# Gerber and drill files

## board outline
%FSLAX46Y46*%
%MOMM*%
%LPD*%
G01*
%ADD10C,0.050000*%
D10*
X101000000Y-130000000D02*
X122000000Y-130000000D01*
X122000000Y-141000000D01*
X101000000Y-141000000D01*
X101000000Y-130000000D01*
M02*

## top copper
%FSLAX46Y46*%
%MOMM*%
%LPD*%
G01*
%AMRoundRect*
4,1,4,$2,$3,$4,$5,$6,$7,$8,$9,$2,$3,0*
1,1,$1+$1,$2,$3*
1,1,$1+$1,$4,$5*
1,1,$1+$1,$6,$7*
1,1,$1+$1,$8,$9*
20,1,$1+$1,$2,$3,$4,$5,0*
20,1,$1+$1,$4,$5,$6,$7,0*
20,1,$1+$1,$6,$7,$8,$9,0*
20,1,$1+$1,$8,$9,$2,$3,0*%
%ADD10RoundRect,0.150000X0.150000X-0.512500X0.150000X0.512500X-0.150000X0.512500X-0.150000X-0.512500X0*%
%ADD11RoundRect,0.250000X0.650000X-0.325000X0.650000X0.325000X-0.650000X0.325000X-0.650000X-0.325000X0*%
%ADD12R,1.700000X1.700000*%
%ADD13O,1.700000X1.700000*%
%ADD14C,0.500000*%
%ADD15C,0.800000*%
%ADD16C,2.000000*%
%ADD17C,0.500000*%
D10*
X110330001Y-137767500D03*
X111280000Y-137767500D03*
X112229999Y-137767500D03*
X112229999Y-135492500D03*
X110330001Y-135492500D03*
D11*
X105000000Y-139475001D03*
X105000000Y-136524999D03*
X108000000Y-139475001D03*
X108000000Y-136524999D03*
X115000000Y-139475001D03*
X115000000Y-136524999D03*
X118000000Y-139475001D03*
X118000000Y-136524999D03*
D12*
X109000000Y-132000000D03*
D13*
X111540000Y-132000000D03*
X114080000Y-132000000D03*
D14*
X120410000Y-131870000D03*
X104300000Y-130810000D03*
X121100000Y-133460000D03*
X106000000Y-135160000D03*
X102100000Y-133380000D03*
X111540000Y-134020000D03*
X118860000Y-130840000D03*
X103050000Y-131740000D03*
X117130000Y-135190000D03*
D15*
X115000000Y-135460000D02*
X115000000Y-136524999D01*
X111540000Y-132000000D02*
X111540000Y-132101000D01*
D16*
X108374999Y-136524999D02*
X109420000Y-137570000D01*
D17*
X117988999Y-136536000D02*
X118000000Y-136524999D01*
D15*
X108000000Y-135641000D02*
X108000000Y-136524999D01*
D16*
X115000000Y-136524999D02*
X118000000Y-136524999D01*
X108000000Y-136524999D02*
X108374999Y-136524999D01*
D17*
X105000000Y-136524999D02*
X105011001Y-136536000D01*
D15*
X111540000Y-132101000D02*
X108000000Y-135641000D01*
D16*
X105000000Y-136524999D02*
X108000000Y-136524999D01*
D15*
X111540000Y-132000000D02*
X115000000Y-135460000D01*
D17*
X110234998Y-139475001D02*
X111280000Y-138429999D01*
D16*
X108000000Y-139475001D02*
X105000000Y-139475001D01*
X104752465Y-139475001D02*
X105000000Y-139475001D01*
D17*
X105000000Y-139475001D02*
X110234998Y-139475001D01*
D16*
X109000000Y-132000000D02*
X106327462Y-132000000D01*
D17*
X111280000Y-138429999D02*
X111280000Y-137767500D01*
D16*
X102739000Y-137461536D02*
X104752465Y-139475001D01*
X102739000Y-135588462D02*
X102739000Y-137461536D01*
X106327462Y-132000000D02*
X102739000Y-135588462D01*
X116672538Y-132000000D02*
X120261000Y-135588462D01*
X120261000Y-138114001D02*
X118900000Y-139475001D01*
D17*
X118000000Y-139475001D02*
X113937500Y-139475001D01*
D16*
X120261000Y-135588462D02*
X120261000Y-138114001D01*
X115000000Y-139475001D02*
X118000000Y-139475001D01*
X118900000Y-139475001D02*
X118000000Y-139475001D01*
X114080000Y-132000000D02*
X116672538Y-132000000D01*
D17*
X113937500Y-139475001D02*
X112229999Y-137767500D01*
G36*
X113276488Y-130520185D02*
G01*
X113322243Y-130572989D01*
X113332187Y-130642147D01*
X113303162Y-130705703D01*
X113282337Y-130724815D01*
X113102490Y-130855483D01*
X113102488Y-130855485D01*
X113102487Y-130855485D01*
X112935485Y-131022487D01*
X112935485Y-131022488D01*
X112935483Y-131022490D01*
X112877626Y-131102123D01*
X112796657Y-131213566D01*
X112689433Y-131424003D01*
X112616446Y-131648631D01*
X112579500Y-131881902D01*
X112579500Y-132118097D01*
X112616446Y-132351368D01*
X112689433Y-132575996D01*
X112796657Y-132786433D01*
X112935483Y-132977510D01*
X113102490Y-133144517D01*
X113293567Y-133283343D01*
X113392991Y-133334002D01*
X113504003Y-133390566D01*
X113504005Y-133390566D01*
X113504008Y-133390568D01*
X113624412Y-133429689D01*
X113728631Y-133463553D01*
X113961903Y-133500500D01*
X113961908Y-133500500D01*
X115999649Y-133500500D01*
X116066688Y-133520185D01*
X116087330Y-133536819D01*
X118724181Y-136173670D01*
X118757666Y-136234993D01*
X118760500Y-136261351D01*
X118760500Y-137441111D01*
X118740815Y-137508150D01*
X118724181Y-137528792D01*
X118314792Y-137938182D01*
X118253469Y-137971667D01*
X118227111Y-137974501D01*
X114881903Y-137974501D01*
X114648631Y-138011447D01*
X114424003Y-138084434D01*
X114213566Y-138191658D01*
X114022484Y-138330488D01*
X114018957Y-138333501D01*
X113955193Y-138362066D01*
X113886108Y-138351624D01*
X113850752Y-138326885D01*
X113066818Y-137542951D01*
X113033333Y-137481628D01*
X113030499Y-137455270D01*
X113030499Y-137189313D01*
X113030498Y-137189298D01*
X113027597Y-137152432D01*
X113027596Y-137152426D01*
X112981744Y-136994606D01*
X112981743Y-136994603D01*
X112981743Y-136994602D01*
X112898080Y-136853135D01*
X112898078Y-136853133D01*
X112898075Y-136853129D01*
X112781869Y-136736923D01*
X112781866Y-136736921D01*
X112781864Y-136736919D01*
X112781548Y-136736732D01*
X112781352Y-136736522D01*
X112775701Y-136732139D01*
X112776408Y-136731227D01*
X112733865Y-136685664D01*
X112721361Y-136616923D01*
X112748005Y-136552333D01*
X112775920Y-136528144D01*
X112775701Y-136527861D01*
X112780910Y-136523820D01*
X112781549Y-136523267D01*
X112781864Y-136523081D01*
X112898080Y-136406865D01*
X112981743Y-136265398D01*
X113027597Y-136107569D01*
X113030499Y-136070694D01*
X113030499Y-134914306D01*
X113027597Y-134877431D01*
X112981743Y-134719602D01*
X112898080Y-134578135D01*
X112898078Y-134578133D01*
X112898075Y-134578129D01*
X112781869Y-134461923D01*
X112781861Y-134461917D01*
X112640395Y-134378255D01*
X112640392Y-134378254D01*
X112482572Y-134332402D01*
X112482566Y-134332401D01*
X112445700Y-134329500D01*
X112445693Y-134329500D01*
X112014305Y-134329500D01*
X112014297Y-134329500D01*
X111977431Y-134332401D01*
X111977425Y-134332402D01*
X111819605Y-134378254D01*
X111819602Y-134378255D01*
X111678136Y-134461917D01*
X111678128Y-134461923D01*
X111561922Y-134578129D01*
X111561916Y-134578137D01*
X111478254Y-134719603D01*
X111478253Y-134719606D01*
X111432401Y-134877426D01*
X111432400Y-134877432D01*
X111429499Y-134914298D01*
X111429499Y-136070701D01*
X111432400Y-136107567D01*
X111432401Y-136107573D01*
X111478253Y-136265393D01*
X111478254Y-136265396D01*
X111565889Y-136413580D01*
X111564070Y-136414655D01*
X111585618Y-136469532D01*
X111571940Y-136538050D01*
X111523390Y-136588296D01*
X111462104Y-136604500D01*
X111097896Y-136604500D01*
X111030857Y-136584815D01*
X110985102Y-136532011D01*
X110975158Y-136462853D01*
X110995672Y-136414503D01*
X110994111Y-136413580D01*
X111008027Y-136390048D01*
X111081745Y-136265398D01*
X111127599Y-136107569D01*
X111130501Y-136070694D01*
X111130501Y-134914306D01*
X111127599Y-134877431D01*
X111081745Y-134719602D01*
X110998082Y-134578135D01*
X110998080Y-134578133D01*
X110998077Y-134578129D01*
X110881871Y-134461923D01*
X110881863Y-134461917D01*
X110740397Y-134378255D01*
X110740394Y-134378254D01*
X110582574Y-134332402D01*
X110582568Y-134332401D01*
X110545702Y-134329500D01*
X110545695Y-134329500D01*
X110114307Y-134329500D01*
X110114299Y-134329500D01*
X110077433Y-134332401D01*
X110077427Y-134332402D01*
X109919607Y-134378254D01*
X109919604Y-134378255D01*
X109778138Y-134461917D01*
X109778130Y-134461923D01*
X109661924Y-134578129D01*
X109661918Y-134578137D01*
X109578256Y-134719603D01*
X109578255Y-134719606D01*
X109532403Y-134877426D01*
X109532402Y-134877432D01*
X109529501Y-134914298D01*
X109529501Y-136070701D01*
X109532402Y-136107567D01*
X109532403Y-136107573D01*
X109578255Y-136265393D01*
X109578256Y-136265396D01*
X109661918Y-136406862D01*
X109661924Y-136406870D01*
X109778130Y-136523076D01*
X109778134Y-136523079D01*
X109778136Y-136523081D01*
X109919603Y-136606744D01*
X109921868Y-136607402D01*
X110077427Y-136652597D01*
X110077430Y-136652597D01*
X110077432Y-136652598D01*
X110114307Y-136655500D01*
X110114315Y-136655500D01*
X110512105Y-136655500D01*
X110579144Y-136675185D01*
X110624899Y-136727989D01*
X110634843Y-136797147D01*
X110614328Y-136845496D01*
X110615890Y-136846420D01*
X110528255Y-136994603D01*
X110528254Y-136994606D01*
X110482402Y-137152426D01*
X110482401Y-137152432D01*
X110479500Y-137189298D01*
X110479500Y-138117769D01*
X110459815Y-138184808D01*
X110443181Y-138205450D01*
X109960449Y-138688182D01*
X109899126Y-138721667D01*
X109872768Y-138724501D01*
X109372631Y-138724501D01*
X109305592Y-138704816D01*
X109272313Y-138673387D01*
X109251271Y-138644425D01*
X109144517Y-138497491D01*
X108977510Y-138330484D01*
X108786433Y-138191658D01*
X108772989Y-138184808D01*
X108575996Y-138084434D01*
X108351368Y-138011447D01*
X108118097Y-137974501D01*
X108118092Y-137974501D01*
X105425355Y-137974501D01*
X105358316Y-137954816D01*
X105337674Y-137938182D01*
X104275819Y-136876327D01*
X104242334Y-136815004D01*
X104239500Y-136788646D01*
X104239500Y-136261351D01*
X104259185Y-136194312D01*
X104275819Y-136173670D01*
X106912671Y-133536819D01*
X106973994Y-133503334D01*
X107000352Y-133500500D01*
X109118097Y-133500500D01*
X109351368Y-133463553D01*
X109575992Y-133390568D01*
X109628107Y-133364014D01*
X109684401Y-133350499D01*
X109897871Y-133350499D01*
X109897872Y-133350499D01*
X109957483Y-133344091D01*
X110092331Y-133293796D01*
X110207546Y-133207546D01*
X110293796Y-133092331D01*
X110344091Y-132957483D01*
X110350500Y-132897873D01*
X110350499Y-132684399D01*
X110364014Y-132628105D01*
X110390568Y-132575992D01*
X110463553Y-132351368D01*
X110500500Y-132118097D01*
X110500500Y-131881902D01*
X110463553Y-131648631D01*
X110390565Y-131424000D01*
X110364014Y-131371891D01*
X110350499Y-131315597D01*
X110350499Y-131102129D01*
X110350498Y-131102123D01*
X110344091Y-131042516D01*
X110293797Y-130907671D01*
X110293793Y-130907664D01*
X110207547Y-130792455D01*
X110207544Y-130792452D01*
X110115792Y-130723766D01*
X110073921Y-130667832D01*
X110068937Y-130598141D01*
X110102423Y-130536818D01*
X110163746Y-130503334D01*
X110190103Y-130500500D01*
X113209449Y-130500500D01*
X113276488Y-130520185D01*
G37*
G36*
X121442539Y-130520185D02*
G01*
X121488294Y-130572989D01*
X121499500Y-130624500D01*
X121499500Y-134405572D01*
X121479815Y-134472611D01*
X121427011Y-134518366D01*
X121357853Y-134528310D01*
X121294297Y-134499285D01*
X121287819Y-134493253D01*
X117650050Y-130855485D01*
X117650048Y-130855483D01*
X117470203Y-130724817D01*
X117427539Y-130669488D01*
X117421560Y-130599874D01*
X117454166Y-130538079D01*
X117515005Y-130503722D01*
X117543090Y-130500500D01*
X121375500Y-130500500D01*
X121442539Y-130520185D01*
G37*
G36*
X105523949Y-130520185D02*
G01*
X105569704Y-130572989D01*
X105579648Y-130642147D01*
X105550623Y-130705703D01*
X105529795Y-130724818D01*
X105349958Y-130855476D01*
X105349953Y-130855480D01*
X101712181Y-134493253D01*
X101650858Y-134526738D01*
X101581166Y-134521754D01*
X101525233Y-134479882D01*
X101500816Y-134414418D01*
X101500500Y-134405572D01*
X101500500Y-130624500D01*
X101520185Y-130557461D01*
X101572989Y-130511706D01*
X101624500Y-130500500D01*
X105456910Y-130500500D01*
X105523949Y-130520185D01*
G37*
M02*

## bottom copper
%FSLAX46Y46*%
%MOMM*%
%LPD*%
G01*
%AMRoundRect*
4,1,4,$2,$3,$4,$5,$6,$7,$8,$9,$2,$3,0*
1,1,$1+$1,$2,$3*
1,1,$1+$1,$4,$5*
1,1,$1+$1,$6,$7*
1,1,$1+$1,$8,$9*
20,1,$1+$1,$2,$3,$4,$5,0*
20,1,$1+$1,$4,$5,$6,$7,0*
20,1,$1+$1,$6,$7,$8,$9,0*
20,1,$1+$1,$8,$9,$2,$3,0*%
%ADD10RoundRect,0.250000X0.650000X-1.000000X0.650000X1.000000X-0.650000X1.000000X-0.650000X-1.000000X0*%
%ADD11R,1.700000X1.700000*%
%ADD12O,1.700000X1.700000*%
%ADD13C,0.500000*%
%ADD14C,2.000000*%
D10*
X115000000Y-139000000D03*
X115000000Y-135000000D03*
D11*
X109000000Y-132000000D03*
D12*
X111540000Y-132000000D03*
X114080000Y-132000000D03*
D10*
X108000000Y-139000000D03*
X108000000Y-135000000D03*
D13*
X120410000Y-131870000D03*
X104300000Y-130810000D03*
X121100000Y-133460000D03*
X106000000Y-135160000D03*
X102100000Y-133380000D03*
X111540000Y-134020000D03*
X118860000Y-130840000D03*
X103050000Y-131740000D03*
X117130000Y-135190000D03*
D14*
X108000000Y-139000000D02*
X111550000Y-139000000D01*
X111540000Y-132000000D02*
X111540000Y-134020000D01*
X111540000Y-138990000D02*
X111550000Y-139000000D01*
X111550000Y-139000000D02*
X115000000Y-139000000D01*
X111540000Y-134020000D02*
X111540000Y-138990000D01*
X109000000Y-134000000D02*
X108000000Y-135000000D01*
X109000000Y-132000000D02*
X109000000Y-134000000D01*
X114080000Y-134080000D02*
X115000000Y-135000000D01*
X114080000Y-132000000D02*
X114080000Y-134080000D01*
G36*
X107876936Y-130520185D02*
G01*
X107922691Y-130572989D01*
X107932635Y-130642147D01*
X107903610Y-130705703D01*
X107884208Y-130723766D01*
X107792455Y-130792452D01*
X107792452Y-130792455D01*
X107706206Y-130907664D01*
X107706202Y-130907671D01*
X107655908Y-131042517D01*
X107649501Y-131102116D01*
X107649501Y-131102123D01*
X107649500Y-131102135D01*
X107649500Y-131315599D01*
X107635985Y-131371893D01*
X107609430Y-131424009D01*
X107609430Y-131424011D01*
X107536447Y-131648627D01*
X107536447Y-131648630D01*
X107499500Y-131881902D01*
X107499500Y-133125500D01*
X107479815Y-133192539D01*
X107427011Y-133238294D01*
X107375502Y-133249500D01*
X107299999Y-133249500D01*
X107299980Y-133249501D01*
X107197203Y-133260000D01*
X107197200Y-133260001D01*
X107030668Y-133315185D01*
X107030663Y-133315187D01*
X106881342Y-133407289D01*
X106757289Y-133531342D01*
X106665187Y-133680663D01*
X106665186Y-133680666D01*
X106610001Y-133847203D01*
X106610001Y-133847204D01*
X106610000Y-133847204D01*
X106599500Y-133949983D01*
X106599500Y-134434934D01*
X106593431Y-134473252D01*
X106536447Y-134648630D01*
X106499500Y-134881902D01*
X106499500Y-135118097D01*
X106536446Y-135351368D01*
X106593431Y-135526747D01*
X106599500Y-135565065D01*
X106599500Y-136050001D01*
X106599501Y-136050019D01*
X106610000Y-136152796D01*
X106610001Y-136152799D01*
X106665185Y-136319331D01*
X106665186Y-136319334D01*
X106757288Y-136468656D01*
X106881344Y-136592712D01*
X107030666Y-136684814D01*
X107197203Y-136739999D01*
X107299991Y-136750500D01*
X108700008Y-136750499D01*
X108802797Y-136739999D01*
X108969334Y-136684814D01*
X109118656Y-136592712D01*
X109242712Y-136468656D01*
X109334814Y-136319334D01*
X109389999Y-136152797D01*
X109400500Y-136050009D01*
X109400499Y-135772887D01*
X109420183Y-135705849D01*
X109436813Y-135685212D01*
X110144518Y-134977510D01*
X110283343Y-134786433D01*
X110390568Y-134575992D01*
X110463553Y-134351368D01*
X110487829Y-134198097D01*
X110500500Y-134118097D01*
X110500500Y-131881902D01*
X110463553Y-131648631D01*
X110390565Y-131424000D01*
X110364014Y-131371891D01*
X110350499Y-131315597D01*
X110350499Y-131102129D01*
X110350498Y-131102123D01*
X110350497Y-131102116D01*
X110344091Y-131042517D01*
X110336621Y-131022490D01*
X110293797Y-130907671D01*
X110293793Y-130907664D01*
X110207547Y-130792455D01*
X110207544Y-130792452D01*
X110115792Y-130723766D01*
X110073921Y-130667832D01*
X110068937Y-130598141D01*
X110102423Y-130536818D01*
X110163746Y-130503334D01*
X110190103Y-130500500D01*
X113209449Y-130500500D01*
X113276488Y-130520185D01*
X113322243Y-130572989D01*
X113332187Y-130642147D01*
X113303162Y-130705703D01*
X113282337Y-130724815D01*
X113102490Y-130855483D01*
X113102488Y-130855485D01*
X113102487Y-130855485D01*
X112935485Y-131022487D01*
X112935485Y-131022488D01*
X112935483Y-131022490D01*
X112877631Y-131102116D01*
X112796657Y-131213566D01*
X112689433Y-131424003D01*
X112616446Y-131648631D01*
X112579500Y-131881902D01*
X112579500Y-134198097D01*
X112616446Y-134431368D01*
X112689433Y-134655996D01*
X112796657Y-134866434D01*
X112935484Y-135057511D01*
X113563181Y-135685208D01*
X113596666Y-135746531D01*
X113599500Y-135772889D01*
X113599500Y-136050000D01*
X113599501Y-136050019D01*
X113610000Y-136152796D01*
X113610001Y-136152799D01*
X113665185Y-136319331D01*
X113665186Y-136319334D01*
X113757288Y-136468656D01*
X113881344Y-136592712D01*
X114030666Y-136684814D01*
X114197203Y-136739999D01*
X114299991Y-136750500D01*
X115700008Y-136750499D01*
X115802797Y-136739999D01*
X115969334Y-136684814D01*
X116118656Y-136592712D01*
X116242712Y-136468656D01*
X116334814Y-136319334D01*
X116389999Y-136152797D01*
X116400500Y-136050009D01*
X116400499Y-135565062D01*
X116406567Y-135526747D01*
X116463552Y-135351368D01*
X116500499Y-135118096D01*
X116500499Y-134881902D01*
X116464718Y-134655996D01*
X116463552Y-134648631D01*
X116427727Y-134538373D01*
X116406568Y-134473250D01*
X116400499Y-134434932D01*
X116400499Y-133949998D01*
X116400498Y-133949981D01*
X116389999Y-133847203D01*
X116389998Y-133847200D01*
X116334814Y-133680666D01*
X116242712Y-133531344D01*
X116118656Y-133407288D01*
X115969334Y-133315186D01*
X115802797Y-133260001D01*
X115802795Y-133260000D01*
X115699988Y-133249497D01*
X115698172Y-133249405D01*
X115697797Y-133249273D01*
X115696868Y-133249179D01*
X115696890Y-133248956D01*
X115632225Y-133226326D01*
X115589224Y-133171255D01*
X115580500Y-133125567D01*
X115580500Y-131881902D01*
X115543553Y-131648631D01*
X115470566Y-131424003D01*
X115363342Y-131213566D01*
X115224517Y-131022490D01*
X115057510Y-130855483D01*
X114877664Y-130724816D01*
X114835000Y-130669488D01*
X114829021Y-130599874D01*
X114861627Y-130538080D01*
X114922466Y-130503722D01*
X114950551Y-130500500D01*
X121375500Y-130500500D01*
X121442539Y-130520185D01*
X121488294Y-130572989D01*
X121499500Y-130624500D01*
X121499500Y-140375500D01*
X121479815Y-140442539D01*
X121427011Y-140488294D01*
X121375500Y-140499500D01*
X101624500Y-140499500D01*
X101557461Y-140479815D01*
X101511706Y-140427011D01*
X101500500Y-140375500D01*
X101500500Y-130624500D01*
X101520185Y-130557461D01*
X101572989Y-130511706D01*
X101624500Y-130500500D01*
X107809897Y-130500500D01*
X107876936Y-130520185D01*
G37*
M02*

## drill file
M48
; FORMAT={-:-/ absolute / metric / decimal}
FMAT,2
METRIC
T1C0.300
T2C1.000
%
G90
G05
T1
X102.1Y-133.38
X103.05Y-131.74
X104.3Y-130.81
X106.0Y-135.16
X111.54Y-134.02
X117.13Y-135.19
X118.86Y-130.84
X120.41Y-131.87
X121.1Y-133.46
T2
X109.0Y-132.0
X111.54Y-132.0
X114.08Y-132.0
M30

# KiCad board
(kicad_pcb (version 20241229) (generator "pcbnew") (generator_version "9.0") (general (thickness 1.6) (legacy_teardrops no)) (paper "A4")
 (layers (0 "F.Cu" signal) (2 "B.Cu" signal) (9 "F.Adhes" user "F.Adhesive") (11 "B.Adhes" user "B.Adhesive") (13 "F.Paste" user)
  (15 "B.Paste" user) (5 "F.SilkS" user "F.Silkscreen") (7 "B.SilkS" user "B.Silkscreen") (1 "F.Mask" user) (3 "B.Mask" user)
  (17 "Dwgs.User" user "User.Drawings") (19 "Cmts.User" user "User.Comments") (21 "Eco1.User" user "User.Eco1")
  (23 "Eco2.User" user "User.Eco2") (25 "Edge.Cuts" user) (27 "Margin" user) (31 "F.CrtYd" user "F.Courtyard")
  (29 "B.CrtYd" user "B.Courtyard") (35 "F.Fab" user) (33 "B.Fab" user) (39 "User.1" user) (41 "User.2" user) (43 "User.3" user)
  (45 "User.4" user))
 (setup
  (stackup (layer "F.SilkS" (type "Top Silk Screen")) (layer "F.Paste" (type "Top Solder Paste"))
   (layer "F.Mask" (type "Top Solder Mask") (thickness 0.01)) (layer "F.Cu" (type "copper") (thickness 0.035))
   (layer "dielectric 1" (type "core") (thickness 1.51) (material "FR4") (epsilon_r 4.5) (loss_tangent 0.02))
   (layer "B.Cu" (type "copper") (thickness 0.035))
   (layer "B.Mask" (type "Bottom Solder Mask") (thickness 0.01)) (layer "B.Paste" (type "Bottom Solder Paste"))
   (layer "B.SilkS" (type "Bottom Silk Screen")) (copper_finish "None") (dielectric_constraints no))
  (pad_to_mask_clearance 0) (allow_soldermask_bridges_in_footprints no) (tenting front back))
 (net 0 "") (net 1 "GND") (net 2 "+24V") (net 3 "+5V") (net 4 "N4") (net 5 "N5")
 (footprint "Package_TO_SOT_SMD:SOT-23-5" (layer "F.Cu") (at 111.28 136.63 90)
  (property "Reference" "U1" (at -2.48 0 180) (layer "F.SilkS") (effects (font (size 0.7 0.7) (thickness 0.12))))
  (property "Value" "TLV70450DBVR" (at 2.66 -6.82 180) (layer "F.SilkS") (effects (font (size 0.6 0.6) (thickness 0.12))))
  (pad "1" smd roundrect (at -1.1375 -0.949999 90) (size 1.325 0.6) (layers "F.Cu" "F.Mask" "F.Paste") (roundrect_rratio 0.25) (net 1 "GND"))
  (pad "2" smd roundrect (at -1.1375 0 90) (size 1.325 0.6) (layers "F.Cu" "F.Mask" "F.Paste") (roundrect_rratio 0.25) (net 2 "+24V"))
  (pad "3" smd roundrect (at -1.1375 0.949999 90) (size 1.325 0.6) (layers "F.Cu" "F.Mask" "F.Paste") (roundrect_rratio 0.25) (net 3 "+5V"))
  (pad "4" smd roundrect (at 1.1375 0.949999 90) (size 1.325 0.6) (layers "F.Cu" "F.Mask" "F.Paste") (roundrect_rratio 0.25) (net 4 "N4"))
  (pad "5" smd roundrect (at 1.1375 -0.949999 90) (size 1.325 0.6) (layers "F.Cu" "F.Mask" "F.Paste") (roundrect_rratio 0.25) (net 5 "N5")))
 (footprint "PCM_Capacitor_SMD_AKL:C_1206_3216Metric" (layer "F.Cu") (at 105 138 90)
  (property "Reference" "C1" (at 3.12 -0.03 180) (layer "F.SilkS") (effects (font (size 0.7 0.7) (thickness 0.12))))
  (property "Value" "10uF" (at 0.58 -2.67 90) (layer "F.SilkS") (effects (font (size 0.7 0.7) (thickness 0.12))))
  (pad "1" smd roundrect (at -1.475001 0 90) (size 1.15 1.8) (layers "F.Cu" "F.Mask" "F.Paste") (roundrect_rratio 0.217391) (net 2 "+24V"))
  (pad "2" smd roundrect (at 1.475001 0 90) (size 1.15 1.8) (layers "F.Cu" "F.Mask" "F.Paste") (roundrect_rratio 0.217391) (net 1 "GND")))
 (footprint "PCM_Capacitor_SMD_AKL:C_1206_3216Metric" (layer "F.Cu") (at 108 138 90)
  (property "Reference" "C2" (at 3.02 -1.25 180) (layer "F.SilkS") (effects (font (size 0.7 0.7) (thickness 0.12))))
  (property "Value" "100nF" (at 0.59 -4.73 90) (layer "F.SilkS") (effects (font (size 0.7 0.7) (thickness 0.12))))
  (pad "1" smd roundrect (at -1.475001 0 90) (size 1.15 1.8) (layers "F.Cu" "F.Mask" "F.Paste") (roundrect_rratio 0.217391) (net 2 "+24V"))
  (pad "2" smd roundrect (at 1.475001 0 90) (size 1.15 1.8) (layers "F.Cu" "F.Mask" "F.Paste") (roundrect_rratio 0.217391) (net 1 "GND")))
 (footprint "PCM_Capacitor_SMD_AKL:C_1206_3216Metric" (layer "F.Cu") (at 115 138 90)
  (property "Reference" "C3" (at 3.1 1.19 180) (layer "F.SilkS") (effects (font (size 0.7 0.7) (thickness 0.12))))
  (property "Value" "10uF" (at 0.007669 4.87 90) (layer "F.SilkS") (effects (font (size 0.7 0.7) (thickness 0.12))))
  (pad "1" smd roundrect (at -1.475001 0 90) (size 1.15 1.8) (layers "F.Cu" "F.Mask" "F.Paste") (roundrect_rratio 0.217391) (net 3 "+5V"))
  (pad "2" smd roundrect (at 1.475001 0 90) (size 1.15 1.8) (layers "F.Cu" "F.Mask" "F.Paste") (roundrect_rratio 0.217391) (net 1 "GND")))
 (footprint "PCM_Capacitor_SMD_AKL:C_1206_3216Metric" (layer "F.Cu") (at 118 138 90)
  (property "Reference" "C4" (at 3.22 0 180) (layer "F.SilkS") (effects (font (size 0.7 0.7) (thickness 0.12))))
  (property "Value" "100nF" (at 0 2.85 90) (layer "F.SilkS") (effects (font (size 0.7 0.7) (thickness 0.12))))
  (pad "1" smd roundrect (at -1.475001 0 90) (size 1.15 1.8) (layers "F.Cu" "F.Mask" "F.Paste") (roundrect_rratio 0.217391) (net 3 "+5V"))
  (pad "2" smd roundrect (at 1.475001 0 90) (size 1.15 1.8) (layers "F.Cu" "F.Mask" "F.Paste") (roundrect_rratio 0.217391) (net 1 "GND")))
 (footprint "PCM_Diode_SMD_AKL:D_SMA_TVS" (layer "B.Cu") (at 115 137 90)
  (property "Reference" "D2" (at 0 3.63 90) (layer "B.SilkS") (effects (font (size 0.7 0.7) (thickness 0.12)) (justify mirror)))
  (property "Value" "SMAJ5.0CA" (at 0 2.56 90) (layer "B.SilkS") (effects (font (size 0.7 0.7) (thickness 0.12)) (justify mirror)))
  (pad "1" smd roundrect (at -2 0 90) (size 2.5 1.8) (layers "B.Cu" "B.Mask" "B.Paste") (roundrect_rratio 0.1388888889) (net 1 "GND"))
  (pad "2" smd roundrect (at 2 0 90) (size 2.5 1.8) (layers "B.Cu" "B.Mask" "B.Paste") (roundrect_rratio 0.1388888889) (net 3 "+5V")))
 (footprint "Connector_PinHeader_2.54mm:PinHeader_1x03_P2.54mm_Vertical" (layer "B.Cu") (at 109 132 -90)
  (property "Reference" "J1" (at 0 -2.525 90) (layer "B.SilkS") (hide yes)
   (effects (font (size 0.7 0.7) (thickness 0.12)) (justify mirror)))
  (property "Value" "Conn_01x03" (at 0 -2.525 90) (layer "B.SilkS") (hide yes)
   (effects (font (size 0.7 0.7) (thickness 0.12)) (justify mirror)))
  (pad "1" thru_hole rect (at 0 0 270) (size 1.7 1.7) (drill 1) (layers "*.Cu" "*.Mask") (remove_unused_layers no) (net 2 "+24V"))
  (pad "2" thru_hole oval (at 0 -2.54 270) (size 1.7 1.7) (drill 1) (layers "*.Cu" "*.Mask") (remove_unused_layers no) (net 1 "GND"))
  (pad "3" thru_hole oval (at 0 -5.08 270) (size 1.7 1.7) (drill 1) (layers "*.Cu" "*.Mask") (remove_unused_layers no) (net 3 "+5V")))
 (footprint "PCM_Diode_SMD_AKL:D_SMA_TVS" (layer "B.Cu") (at 108 137 90)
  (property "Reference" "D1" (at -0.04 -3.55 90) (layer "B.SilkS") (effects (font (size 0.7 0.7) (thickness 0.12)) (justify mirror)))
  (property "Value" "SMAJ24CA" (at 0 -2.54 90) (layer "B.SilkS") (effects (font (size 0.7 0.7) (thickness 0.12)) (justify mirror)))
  (pad "1" smd roundrect (at -2 0 90) (size 2.5 1.8) (layers "B.Cu" "B.Mask" "B.Paste") (roundrect_rratio 0.1388888889) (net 1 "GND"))
  (pad "2" smd roundrect (at 2 0 90) (size 2.5 1.8) (layers "B.Cu" "B.Mask" "B.Paste") (roundrect_rratio 0.1388888889) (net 2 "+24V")))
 (gr_rect (start 101 130) (end 122 141) (stroke (width 0.05) (type default)) (fill no) (locked yes) (layer "Edge.Cuts"))
 (segment (start 115 135.46) (end 115 136.524999) (width 0.8) (layer "F.Cu") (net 1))
 (segment (start 111.54 132) (end 111.54 132.101) (width 0.8) (layer "F.Cu") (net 1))
 (segment (start 108.374999 136.524999) (end 109.42 137.57) (width 2) (layer "F.Cu") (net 1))
 (segment (start 117.988999 136.536) (end 118 136.524999) (width 0.5) (layer "F.Cu") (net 1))
 (segment (start 108 135.641) (end 108 136.524999) (width 0.8) (layer "F.Cu") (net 1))
 (segment (start 115 136.524999) (end 118 136.524999) (width 2) (layer "F.Cu") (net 1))
 (segment (start 108 136.524999) (end 108.374999 136.524999) (width 2) (layer "F.Cu") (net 1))
 (segment (start 105 136.524999) (end 105.011001 136.536) (width 0.5) (layer "F.Cu") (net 1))
 (segment (start 111.54 132.101) (end 108 135.641) (width 0.8) (layer "F.Cu") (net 1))
 (segment (start 105 136.524999) (end 108 136.524999) (width 2) (layer "F.Cu") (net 1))
 (segment (start 111.54 132) (end 115 135.46) (width 0.8) (layer "F.Cu") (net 1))
 (via (at 120.41 131.87) (size 0.5) (drill 0.3) (layers "F.Cu" "B.Cu") (free yes) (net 1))
 (via (at 104.3 130.81) (size 0.5) (drill 0.3) (layers "F.Cu" "B.Cu") (free yes) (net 1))
 (via (at 121.1 133.46) (size 0.5) (drill 0.3) (layers "F.Cu" "B.Cu") (free yes) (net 1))
 (via (at 106 135.16) (size 0.5) (drill 0.3) (layers "F.Cu" "B.Cu") (free yes) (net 1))
 (via (at 102.1 133.38) (size 0.5) (drill 0.3) (layers "F.Cu" "B.Cu") (free yes) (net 1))
 (via (at 111.54 134.02) (size 0.5) (drill 0.3) (layers "F.Cu" "B.Cu") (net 1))
 (via (at 118.86 130.84) (size 0.5) (drill 0.3) (layers "F.Cu" "B.Cu") (free yes) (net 1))
 (via (at 103.05 131.74) (size 0.5) (drill 0.3) (layers "F.Cu" "B.Cu") (free yes) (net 1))
 (via (at 117.13 135.19) (size 0.5) (drill 0.3) (layers "F.Cu" "B.Cu") (free yes) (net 1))
 (segment (start 108 139) (end 111.55 139) (width 2) (layer "B.Cu") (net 1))
 (segment (start 111.54 132) (end 111.54 134.02) (width 2) (layer "B.Cu") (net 1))
 (segment (start 111.54 138.99) (end 111.55 139) (width 2) (layer "B.Cu") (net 1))
 (segment (start 111.55 139) (end 115 139) (width 2) (layer "B.Cu") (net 1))
 (segment (start 111.54 134.02) (end 111.54 138.99) (width 2) (layer "B.Cu") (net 1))
 (segment (start 110.234998 139.475001) (end 111.28 138.429999) (width 0.5) (layer "F.Cu") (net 2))
 (segment (start 108 139.475001) (end 105 139.475001) (width 2) (layer "F.Cu") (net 2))
 (segment (start 104.752465 139.475001) (end 105 139.475001) (width 2) (layer "F.Cu") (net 2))
 (segment (start 105 139.475001) (end 110.234998 139.475001) (width 0.5) (layer "F.Cu") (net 2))
 (segment (start 109 132) (end 106.327462 132) (width 2) (layer "F.Cu") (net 2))
 (segment (start 111.28 138.429999) (end 111.28 137.7675) (width 0.5) (layer "F.Cu") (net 2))
 (segment (start 102.739 137.461536) (end 104.752465 139.475001) (width 2) (layer "F.Cu") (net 2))
 (segment (start 102.739 135.588462) (end 102.739 137.461536) (width 2) (layer "F.Cu") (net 2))
 (segment (start 106.327462 132) (end 102.739 135.588462) (width 2) (layer "F.Cu") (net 2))
 (segment (start 109 134) (end 108 135) (width 2) (layer "B.Cu") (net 2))
 (segment (start 109 132) (end 109 134) (width 2) (layer "B.Cu") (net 2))
 (segment (start 116.672538 132) (end 120.261 135.588462) (width 2) (layer "F.Cu") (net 3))
 (segment (start 120.261 138.114001) (end 118.9 139.475001) (width 2) (layer "F.Cu") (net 3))
 (segment (start 118 139.475001) (end 113.9375 139.475001) (width 0.5) (layer "F.Cu") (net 3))
 (segment (start 120.261 135.588462) (end 120.261 138.114001) (width 2) (layer "F.Cu") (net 3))
 (segment (start 115 139.475001) (end 118 139.475001) (width 2) (layer "F.Cu") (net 3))
 (segment (start 118.9 139.475001) (end 118 139.475001) (width 2) (layer "F.Cu") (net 3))
 (segment (start 114.08 132) (end 116.672538 132) (width 2) (layer "F.Cu") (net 3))
 (segment (start 113.9375 139.475001) (end 112.229999 137.7675) (width 0.5) (layer "F.Cu") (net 3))
 (segment (start 114.08 134.08) (end 115 135) (width 2) (layer "B.Cu") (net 3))
 (segment (start 114.08 132) (end 114.08 134.08) (width 2) (layer "B.Cu") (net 3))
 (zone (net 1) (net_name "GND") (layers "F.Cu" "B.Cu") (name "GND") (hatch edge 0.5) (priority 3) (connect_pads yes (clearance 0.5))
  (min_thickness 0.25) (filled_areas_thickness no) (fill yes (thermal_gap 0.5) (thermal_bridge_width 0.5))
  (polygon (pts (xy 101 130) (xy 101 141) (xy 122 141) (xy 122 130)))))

